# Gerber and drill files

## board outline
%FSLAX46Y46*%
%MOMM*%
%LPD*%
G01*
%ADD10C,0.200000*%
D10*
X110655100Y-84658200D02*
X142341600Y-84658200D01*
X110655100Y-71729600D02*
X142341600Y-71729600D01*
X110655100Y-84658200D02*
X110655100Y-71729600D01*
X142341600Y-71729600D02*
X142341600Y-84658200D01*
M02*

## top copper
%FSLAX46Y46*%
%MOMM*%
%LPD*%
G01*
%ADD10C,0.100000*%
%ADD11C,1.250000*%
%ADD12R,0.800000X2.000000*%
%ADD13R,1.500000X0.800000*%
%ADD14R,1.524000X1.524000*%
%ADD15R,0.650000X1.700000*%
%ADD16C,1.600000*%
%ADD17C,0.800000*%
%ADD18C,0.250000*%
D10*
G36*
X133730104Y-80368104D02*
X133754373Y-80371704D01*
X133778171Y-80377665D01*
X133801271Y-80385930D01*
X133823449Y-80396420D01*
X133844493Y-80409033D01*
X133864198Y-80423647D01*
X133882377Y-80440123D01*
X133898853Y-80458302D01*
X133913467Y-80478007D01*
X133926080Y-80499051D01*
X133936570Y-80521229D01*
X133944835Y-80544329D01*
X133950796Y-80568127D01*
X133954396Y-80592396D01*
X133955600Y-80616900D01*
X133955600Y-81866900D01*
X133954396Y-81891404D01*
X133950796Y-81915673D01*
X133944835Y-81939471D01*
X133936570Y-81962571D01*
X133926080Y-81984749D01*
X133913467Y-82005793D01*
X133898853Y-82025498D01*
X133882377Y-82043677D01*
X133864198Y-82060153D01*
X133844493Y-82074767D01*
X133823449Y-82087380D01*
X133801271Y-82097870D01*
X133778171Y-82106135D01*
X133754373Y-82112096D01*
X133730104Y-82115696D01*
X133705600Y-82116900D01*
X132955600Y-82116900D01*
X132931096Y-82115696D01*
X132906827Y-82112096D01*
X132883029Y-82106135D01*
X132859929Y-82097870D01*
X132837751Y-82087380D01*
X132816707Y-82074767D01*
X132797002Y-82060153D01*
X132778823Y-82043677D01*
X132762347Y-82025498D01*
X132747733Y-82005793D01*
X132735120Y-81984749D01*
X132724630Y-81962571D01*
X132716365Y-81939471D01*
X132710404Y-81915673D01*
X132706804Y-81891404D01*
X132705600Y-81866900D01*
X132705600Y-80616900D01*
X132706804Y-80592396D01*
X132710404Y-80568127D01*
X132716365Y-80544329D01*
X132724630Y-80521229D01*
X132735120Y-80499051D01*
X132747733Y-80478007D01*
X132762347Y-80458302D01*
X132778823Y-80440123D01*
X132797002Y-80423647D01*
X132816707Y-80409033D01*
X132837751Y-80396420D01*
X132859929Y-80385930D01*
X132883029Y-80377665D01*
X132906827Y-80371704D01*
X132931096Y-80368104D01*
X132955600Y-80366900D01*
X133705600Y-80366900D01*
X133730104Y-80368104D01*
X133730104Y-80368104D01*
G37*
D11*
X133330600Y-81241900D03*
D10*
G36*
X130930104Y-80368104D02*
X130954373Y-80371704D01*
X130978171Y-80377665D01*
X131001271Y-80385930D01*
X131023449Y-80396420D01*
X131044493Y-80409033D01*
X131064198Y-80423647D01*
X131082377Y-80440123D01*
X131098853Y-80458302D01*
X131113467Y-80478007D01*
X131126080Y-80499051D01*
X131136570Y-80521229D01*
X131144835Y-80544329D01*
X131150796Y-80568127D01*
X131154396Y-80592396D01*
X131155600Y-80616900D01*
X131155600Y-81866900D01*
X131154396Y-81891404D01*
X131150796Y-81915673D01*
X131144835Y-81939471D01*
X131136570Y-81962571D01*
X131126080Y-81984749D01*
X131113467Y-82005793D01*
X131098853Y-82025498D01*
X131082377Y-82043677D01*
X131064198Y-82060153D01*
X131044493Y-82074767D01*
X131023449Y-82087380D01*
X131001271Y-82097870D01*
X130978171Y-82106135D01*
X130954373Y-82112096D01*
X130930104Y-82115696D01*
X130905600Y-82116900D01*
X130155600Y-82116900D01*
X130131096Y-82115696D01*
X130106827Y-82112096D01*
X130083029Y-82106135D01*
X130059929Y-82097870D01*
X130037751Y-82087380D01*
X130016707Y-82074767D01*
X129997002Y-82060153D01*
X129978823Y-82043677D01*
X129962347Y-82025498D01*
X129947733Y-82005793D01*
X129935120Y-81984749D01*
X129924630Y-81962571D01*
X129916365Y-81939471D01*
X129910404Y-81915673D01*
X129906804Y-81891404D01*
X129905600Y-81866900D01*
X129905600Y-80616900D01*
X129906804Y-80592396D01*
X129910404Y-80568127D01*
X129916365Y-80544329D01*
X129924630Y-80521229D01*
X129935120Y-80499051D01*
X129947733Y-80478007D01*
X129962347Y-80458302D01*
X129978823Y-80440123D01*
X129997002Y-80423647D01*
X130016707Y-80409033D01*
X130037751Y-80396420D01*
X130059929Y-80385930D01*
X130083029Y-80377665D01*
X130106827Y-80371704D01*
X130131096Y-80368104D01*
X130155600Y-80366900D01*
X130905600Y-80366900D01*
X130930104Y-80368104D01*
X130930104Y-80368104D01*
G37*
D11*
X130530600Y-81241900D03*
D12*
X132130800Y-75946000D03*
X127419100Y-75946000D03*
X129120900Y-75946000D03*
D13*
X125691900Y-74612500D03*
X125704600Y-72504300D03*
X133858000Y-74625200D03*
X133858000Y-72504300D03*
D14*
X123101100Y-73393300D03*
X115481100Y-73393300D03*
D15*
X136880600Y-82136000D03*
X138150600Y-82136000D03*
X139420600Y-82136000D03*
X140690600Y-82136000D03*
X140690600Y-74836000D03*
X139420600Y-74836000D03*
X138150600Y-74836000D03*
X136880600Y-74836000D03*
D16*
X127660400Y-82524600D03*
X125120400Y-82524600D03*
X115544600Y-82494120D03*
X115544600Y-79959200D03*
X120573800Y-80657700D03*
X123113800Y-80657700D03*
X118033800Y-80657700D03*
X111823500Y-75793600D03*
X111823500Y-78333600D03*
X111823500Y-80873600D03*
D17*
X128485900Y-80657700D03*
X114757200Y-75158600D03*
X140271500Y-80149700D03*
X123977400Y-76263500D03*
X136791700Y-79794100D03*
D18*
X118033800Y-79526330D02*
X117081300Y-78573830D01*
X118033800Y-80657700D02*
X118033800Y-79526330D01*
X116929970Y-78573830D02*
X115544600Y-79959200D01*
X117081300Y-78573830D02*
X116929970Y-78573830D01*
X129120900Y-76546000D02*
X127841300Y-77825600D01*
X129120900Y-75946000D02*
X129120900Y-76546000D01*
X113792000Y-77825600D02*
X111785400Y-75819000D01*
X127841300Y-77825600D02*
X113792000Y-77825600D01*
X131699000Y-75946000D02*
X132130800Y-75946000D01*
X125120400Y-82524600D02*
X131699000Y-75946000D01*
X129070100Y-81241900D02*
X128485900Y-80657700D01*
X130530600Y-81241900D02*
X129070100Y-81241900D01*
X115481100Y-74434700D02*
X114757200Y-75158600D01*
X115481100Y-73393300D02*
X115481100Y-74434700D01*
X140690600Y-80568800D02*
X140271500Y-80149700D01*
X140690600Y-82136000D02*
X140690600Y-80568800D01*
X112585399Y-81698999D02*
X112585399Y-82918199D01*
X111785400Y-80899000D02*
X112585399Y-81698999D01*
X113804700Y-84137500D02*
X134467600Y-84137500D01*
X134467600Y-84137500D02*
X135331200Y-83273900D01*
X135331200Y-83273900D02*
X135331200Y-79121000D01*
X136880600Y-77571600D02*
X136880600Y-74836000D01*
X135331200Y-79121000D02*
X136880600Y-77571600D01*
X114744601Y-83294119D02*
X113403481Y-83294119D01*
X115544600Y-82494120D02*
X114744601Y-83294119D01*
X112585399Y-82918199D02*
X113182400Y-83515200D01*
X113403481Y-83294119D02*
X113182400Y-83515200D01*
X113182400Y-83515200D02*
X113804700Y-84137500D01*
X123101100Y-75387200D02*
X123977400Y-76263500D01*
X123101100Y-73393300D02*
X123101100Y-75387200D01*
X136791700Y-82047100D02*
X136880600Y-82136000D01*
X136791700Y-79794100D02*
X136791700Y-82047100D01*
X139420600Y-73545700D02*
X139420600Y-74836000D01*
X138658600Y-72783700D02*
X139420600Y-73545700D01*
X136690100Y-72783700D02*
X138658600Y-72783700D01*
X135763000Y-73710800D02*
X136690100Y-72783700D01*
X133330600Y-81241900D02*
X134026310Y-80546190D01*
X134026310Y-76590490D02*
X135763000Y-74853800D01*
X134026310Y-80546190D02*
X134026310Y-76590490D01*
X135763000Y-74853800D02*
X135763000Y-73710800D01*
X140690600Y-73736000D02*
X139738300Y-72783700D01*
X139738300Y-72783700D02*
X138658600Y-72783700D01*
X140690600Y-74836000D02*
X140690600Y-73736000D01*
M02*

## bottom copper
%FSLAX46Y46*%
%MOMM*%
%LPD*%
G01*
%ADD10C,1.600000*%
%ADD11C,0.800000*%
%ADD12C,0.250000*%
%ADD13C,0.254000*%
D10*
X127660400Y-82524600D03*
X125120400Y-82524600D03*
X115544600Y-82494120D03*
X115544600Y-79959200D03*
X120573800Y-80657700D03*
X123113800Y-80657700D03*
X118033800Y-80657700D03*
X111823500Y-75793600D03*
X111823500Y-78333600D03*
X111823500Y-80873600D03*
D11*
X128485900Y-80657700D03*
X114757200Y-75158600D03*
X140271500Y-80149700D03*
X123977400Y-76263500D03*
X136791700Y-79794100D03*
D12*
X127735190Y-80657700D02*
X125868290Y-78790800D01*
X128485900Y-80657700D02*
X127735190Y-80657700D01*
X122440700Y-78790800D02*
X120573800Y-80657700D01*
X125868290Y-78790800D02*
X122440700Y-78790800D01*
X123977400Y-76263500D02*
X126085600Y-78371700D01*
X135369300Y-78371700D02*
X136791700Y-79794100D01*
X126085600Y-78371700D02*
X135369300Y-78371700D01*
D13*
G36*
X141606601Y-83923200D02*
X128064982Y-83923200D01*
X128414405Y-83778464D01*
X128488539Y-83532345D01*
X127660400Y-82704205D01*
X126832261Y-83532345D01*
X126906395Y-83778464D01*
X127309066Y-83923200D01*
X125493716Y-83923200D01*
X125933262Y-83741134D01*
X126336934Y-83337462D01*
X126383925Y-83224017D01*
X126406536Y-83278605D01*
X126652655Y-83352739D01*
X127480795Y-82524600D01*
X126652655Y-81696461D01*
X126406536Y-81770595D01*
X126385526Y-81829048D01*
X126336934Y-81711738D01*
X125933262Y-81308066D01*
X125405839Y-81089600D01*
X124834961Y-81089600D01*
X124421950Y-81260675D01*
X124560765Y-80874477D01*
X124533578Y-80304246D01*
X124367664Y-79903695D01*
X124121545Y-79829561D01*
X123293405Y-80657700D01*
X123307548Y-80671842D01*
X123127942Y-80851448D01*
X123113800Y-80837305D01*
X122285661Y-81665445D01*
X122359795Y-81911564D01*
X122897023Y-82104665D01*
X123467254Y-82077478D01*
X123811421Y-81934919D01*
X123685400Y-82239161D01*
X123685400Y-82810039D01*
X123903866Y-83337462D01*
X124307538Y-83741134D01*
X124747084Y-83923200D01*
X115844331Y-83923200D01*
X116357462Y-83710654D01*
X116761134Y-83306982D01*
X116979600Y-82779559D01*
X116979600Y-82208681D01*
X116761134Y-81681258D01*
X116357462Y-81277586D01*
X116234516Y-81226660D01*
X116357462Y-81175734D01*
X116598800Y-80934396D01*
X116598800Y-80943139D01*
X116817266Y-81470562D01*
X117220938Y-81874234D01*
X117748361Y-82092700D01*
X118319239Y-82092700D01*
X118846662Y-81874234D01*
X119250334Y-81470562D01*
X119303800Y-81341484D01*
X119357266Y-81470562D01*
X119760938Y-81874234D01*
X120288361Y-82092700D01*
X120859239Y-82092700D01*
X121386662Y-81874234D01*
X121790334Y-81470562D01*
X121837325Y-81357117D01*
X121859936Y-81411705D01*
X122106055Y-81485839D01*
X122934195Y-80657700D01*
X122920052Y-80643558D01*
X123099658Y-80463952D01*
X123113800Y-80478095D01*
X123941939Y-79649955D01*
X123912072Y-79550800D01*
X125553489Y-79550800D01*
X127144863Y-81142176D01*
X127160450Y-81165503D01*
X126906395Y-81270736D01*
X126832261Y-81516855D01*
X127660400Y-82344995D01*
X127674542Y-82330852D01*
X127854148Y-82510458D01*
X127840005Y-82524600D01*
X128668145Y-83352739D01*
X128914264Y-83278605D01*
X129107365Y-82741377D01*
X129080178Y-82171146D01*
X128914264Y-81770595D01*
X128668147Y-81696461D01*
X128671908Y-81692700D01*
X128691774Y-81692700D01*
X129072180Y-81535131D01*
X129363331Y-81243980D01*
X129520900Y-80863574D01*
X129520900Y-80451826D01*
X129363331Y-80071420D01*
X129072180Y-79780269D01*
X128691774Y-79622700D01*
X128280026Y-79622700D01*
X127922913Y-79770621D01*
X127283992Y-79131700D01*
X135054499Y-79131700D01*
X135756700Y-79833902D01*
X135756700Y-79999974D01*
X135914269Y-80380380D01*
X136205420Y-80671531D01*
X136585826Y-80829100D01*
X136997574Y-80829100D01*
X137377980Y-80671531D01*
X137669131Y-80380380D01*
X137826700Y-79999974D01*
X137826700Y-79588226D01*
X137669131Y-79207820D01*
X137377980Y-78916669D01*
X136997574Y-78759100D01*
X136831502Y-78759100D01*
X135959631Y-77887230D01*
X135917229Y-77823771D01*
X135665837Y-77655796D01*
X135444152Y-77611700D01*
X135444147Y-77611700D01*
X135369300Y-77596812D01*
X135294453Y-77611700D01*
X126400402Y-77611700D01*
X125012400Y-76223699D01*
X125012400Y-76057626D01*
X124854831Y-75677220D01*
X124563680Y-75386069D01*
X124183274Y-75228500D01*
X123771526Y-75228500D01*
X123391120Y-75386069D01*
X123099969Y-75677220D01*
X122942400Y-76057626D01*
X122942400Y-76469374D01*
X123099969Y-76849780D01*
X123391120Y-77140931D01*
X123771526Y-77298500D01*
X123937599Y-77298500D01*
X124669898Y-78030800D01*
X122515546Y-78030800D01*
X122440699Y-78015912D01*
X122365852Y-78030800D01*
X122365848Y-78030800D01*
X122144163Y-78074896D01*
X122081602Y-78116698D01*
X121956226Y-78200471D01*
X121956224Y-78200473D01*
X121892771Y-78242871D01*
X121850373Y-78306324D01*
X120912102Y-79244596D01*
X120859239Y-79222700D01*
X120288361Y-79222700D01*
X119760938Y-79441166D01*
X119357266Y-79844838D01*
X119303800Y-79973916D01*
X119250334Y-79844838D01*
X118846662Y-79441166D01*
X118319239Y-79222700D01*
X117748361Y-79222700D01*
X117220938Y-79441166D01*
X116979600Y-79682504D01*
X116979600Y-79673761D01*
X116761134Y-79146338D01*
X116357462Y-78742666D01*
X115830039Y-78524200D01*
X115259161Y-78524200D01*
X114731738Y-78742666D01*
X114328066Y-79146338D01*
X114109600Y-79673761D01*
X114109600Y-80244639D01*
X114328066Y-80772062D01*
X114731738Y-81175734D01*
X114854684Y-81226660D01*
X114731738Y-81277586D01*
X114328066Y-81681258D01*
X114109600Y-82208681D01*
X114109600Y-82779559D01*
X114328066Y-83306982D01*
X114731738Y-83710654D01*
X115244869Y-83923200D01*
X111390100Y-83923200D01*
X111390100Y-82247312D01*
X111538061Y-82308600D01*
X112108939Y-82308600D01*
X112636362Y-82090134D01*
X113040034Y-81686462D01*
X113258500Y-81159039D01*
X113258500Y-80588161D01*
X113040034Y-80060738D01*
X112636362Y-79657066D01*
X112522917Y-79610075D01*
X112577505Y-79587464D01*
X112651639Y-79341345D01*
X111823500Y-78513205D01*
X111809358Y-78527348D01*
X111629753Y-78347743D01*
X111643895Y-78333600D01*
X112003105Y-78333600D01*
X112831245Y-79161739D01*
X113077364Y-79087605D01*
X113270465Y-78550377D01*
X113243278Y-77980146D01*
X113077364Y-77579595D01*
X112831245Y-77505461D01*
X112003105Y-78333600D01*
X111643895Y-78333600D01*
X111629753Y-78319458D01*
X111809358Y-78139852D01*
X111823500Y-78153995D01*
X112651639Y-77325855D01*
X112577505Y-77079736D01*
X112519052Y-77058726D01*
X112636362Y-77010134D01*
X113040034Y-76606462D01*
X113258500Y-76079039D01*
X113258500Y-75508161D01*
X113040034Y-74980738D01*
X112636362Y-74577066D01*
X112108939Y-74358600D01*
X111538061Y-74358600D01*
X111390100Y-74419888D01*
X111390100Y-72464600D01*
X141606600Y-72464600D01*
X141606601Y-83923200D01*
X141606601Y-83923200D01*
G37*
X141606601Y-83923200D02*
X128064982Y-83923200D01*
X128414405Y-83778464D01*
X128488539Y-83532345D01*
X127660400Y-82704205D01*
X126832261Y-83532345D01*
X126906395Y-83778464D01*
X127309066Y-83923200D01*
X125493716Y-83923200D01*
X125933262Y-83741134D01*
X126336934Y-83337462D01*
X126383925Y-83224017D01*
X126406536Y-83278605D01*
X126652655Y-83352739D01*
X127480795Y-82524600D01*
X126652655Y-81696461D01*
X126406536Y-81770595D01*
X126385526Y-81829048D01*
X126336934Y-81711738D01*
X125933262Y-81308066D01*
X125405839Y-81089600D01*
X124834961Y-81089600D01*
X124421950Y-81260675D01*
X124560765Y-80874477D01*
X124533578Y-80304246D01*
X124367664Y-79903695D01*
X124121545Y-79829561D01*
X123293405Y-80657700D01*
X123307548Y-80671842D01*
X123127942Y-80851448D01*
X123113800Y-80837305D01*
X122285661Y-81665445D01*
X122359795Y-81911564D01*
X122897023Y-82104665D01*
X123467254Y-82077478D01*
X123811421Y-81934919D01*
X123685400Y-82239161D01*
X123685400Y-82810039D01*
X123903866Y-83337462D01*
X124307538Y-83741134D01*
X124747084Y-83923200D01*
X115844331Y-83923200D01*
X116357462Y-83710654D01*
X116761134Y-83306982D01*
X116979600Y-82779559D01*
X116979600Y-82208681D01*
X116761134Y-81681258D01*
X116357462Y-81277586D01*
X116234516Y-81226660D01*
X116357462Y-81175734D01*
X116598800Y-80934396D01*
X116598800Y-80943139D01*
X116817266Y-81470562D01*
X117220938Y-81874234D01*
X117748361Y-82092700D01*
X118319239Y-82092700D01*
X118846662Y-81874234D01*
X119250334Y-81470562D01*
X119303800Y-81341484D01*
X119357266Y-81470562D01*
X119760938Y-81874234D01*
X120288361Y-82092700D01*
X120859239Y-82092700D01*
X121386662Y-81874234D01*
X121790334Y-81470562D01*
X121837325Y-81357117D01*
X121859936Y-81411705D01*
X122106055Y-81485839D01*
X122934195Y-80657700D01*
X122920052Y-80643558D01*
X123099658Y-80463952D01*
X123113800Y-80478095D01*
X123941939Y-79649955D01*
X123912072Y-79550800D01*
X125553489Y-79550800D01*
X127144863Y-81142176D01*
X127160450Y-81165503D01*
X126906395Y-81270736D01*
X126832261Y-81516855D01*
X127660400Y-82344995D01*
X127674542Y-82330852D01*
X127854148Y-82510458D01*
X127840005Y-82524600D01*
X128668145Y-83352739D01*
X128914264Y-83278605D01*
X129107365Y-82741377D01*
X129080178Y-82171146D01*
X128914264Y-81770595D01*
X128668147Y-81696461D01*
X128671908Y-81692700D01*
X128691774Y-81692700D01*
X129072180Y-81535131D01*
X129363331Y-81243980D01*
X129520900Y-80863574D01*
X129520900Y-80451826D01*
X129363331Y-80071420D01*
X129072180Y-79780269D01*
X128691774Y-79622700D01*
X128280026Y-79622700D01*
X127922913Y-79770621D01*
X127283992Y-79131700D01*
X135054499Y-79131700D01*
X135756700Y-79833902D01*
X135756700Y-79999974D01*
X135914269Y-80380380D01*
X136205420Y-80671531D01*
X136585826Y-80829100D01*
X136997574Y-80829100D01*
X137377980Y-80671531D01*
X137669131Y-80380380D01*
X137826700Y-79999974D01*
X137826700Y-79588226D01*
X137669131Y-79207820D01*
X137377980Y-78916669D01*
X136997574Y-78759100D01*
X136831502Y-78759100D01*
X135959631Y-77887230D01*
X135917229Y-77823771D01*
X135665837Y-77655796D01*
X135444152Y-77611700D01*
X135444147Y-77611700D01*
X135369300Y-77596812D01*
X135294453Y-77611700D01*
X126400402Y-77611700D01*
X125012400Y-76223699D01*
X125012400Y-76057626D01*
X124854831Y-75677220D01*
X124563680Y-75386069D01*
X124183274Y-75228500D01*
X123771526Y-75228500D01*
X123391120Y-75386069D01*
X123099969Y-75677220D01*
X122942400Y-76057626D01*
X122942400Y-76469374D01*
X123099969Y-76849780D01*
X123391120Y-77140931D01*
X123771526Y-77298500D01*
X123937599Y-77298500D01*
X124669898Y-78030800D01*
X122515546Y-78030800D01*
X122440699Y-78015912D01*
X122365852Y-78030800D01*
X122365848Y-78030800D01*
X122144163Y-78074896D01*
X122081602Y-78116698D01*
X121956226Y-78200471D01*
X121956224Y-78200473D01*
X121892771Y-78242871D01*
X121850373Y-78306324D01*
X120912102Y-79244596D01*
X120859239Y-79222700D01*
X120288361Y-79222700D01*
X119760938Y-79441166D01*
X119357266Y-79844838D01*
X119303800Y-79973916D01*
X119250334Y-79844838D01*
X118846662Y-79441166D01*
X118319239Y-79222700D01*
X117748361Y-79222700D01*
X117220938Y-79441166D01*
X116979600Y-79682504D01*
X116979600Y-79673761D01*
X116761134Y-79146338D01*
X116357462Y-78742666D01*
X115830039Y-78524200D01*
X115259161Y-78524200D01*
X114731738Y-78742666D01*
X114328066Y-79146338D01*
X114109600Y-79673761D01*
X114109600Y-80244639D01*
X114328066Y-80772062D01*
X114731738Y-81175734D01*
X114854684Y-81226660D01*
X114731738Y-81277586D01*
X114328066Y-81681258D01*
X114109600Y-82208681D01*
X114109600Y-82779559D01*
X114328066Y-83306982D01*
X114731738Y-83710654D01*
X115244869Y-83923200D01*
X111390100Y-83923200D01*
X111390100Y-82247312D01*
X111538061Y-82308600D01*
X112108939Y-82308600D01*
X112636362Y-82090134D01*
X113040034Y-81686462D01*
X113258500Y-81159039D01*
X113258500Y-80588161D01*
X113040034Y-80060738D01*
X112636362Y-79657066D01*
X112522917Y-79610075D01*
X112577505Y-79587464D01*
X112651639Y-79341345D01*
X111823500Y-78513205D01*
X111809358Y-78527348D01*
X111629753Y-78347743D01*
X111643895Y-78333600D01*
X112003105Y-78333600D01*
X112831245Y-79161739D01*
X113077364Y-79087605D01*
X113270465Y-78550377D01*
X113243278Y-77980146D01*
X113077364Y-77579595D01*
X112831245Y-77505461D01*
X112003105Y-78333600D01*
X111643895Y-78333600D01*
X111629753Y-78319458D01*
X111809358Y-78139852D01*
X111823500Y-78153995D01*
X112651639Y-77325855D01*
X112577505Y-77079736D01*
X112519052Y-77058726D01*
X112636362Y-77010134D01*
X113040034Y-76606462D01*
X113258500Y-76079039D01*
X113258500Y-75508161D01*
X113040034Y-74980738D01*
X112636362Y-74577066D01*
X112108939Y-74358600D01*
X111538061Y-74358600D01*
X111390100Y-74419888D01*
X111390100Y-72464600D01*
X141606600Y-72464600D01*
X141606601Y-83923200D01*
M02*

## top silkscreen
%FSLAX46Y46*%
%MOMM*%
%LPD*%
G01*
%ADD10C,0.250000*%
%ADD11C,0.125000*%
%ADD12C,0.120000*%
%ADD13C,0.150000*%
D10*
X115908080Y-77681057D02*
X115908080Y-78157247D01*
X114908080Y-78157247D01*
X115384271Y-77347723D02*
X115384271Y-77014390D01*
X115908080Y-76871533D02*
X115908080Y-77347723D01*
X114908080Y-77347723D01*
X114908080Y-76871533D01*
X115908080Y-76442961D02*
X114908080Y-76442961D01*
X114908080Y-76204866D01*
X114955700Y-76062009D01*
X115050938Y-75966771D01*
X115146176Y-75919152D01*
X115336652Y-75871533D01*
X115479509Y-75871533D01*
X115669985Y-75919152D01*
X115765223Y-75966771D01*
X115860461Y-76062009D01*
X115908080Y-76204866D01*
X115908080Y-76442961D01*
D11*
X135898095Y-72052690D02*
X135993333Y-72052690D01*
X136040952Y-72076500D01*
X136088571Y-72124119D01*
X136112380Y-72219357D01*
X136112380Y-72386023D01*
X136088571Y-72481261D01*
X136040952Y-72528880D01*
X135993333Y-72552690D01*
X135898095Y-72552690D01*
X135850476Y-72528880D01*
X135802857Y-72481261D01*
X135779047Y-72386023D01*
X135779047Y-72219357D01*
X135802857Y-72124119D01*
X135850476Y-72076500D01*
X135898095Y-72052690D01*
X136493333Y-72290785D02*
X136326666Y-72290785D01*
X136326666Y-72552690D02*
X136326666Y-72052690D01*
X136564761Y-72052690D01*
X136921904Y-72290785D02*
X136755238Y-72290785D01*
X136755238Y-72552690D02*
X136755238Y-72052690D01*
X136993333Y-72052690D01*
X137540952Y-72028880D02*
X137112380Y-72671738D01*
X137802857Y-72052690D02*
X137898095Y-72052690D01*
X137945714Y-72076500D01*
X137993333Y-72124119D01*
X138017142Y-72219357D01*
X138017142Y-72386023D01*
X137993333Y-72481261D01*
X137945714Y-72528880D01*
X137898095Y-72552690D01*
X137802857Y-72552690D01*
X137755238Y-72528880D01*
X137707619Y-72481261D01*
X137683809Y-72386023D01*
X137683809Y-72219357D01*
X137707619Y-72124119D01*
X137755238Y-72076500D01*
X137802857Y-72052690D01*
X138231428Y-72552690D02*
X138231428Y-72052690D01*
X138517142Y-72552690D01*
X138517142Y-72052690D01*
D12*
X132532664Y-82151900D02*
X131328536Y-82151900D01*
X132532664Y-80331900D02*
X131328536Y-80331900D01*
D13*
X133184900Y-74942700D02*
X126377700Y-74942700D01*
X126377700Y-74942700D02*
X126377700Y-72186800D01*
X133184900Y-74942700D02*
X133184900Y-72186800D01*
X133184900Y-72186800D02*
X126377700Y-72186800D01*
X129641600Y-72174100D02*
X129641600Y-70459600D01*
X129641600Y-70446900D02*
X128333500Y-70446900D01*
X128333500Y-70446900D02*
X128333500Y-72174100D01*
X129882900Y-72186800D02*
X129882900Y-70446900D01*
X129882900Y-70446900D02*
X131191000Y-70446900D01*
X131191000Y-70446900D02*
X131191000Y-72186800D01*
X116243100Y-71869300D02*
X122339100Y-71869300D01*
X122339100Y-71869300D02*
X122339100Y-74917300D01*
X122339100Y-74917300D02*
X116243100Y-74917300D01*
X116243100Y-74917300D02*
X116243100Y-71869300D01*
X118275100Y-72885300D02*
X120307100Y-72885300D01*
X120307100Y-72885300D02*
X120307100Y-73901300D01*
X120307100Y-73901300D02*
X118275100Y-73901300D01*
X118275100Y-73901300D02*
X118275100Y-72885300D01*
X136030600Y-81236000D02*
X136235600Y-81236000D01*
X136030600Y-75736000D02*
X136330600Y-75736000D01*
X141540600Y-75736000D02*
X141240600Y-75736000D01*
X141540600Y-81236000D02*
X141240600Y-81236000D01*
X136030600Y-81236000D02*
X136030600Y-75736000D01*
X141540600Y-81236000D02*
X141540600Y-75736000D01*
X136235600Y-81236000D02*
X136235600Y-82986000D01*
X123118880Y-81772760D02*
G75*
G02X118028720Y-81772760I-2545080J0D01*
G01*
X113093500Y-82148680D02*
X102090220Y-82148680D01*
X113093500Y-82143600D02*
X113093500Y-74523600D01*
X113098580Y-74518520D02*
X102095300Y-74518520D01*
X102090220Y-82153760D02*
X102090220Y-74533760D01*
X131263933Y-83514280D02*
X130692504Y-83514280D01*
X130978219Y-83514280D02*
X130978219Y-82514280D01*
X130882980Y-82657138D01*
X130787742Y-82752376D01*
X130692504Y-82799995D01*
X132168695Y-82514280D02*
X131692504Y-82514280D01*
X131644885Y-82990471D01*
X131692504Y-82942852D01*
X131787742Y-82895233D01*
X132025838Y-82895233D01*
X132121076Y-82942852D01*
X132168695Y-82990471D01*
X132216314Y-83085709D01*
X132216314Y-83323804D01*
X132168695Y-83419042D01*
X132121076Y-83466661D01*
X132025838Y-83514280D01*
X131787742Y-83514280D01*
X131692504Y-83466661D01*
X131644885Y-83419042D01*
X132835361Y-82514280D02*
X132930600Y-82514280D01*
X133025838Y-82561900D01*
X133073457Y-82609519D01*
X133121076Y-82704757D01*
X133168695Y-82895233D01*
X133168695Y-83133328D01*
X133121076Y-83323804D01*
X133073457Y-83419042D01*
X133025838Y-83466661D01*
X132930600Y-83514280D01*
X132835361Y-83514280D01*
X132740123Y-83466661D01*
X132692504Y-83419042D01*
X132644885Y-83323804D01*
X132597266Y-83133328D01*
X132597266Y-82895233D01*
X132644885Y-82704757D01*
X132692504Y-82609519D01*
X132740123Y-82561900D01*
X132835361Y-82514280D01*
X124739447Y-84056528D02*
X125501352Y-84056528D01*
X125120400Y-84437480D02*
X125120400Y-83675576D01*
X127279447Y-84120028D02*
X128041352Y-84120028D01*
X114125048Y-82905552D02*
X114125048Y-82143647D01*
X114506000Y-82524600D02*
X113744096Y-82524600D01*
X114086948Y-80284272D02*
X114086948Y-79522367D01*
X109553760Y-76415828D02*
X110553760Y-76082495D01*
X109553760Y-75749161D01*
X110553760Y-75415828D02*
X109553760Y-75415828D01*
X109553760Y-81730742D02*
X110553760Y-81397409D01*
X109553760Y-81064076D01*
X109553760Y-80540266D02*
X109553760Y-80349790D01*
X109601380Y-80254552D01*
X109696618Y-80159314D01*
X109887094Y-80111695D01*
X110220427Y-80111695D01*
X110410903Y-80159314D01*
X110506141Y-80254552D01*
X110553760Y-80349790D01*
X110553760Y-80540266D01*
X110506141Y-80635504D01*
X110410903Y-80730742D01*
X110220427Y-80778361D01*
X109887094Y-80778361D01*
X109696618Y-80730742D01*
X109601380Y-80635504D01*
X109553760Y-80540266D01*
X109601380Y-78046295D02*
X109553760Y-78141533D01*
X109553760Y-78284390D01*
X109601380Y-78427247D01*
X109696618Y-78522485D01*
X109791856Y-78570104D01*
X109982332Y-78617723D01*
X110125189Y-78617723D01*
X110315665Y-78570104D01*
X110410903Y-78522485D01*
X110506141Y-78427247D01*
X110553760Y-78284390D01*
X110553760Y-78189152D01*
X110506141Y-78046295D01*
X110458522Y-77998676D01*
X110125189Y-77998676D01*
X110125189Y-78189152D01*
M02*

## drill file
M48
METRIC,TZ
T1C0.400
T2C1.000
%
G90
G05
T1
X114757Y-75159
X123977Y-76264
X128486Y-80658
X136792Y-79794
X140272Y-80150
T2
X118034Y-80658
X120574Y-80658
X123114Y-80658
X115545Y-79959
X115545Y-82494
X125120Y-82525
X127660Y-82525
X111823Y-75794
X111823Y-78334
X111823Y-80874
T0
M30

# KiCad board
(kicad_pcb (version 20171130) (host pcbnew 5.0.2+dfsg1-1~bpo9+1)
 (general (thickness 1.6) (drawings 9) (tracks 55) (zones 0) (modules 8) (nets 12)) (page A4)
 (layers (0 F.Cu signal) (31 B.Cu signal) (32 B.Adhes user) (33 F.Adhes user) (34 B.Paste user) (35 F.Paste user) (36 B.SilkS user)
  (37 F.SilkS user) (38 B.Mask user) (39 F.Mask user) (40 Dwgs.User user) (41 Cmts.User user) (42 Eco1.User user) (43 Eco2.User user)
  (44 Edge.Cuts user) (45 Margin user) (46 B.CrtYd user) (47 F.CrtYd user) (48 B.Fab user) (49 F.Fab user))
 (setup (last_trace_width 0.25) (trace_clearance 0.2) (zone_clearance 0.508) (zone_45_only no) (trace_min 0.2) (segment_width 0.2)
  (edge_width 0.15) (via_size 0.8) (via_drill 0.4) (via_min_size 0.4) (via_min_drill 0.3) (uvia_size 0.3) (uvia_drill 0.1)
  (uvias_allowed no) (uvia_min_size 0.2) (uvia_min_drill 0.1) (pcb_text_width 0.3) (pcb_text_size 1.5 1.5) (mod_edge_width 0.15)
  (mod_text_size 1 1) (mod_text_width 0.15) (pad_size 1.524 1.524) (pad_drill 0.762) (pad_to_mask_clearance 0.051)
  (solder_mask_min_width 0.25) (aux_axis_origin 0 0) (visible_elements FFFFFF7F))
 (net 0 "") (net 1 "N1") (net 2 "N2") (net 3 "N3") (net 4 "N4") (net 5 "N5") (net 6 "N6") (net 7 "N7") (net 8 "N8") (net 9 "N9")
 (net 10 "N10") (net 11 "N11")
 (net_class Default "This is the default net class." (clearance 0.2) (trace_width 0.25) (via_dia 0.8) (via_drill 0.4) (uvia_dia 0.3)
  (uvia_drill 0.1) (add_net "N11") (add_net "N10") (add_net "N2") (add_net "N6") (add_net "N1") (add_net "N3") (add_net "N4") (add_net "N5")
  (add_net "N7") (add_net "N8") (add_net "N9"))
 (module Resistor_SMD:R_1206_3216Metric (layer F.Cu) (at 131.9306 81.2419 180)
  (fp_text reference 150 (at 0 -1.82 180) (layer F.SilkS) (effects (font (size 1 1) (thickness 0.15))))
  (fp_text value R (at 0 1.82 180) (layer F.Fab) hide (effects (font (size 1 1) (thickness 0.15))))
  (fp_line (start -0.602064 -0.91) (end 0.602064 -0.91) (layer F.SilkS) (width 0.12))
  (fp_line (start -0.602064 0.91) (end 0.602064 0.91) (layer F.SilkS) (width 0.12))
  (pad 1 smd roundrect (at -1.4 0 180) (size 1.25 1.75) (layers F.Cu F.Paste F.Mask) (roundrect_rratio 0.2) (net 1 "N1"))
  (pad 2 smd roundrect (at 1.4 0 180) (size 1.25 1.75) (layers F.Cu F.Paste F.Mask) (roundrect_rratio 0.2) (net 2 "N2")))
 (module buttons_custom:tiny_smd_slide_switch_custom (layer F.Cu) (at 132.1308 74.9427 180)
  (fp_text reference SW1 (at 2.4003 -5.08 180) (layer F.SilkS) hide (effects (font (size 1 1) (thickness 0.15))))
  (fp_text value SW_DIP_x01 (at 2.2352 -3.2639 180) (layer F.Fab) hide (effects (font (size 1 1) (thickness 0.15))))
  (fp_line (start -1.0541 0) (end 5.7531 0) (layer F.SilkS) (width 0.15))
  (fp_line (start 5.7531 0) (end 5.7531 2.7559) (layer F.SilkS) (width 0.15))
  (fp_line (start -1.0541 0) (end -1.0541 2.7559) (layer F.SilkS) (width 0.15))
  (fp_line (start -1.0541 2.7559) (end 5.7531 2.7559) (layer F.SilkS) (width 0.15))
  (fp_line (start 2.4892 2.7686) (end 2.4892 4.4831) (layer F.SilkS) (width 0.15))
  (fp_line (start 2.4892 4.4958) (end 3.7973 4.4958) (layer F.SilkS) (width 0.15))
  (fp_line (start 3.7973 4.4958) (end 3.7973 2.7686) (layer F.SilkS) (width 0.15))
  (fp_line (start 2.2479 2.7559) (end 2.2479 4.4958) (layer F.SilkS) (width 0.15))
  (fp_line (start 2.2479 4.4958) (end 0.9398 4.4958) (layer F.SilkS) (width 0.15))
  (fp_line (start 0.9398 4.4958) (end 0.9398 2.7559) (layer F.SilkS) (width 0.15))
  (pad 1 smd rect (at 0 -1.0033 180) (size 0.8 2) (layers F.Cu F.Paste F.Mask) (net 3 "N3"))
  (pad 3 smd rect (at 4.7117 -1.0033 180) (size 0.8 2) (layers F.Cu F.Paste F.Mask))
  (pad 2 smd rect (at 3.0099 -1.0033 180) (size 0.8 2) (layers F.Cu F.Paste F.Mask) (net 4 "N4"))
  (pad 4 smd rect (at 6.4389 0.3302 270) (size 0.8 1.5) (layers F.Cu F.Paste F.Mask))
  (pad 4 smd rect (at 6.4262 2.4384 270) (size 0.8 1.5) (layers F.Cu F.Paste F.Mask))
  (pad 4 smd rect (at -1.7272 0.3175 270) (size 0.8 1.5) (layers F.Cu F.Paste F.Mask))
  (pad 4 smd rect (at -1.7272 2.4384 270) (size 0.8 1.5) (layers F.Cu F.Paste F.Mask)))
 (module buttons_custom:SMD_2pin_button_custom (layer F.Cu) (at 119.2911 73.3933)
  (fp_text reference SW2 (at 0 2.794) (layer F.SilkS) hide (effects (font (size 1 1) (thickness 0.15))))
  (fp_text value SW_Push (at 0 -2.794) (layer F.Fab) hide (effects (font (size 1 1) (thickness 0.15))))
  (fp_line (start -3.048 -1.524) (end 3.048 -1.524) (layer F.SilkS) (width 0.15))
  (fp_line (start 3.048 -1.524) (end 3.048 1.524) (layer F.SilkS) (width 0.15))
  (fp_line (start 3.048 1.524) (end -3.048 1.524) (layer F.SilkS) (width 0.15))
  (fp_line (start -3.048 1.524) (end -3.048 -1.524) (layer F.SilkS) (width 0.15))
  (fp_line (start -1.016 -0.508) (end 1.016 -0.508) (layer F.SilkS) (width 0.15))
  (fp_line (start 1.016 -0.508) (end 1.016 0.508) (layer F.SilkS) (width 0.15))
  (fp_line (start 1.016 0.508) (end -1.016 0.508) (layer F.SilkS) (width 0.15))
  (fp_line (start -1.016 0.508) (end -1.016 -0.508) (layer F.SilkS) (width 0.15))
  (pad 1 smd rect (at 3.81 0) (size 1.524 1.524) (layers F.Cu F.Paste F.Mask) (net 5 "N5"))
  (pad 2 smd rect (at -3.81 0) (size 1.524 1.524) (layers F.Cu F.Paste F.Mask) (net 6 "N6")))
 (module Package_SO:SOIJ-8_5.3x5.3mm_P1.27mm (layer F.Cu) (at 138.7856 78.486 90)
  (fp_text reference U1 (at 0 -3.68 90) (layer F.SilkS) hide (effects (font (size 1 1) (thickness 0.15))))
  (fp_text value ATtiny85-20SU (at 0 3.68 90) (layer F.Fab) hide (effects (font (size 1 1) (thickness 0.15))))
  (fp_line (start -2.75 -2.755) (end -2.75 -2.55) (layer F.SilkS) (width 0.15))
  (fp_line (start 2.75 -2.755) (end 2.75 -2.455) (layer F.SilkS) (width 0.15))
  (fp_line (start 2.75 2.755) (end 2.75 2.455) (layer F.SilkS) (width 0.15))
  (fp_line (start -2.75 2.755) (end -2.75 2.455) (layer F.SilkS) (width 0.15))
  (fp_line (start -2.75 -2.755) (end 2.75 -2.755) (layer F.SilkS) (width 0.15))
  (fp_line (start -2.75 2.755) (end 2.75 2.755) (layer F.SilkS) (width 0.15))
  (fp_line (start -2.75 -2.55) (end -4.5 -2.55) (layer F.SilkS) (width 0.15))
  (pad 1 smd rect (at -3.65 -1.905 90) (size 1.7 0.65) (layers F.Cu F.Paste F.Mask) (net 5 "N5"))
  (pad 2 smd rect (at -3.65 -0.635 90) (size 1.7 0.65) (layers F.Cu F.Paste F.Mask) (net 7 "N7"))
  (pad 3 smd rect (at -3.65 0.635 90) (size 1.7 0.65) (layers F.Cu F.Paste F.Mask) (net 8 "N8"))
  (pad 4 smd rect (at -3.65 1.905 90) (size 1.7 0.65) (layers F.Cu F.Paste F.Mask) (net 6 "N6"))
  (pad 5 smd rect (at 3.65 1.905 90) (size 1.7 0.65) (layers F.Cu F.Paste F.Mask) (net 1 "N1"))
  (pad 6 smd rect (at 3.65 0.635 90) (size 1.7 0.65) (layers F.Cu F.Paste F.Mask) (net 1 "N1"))
  (pad 7 smd rect (at 3.65 -0.635 90) (size 1.7 0.65) (layers F.Cu F.Paste F.Mask) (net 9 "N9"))
  (pad 8 smd rect (at 3.65 -1.905 90) (size 1.7 0.65) (layers F.Cu F.Paste F.Mask) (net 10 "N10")))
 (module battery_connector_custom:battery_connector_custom (layer F.Cu) (at 126.3904 82.5246 180)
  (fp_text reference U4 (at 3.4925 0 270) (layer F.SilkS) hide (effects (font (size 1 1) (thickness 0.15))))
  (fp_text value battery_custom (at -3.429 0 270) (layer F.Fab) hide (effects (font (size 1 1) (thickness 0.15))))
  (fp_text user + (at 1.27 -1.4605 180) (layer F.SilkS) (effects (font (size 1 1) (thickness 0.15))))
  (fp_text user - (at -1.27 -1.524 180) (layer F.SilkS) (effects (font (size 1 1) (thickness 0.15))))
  (pad 1 thru_hole circle (at -1.27 0 180) (size 1.6 1.6) (drill 1) (layers *.Cu *.Mask) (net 6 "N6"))
  (pad 2 thru_hole circle (at 1.27 0 180) (size 1.6 1.6) (drill 1) (layers *.Cu *.Mask) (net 3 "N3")))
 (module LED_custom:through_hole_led (layer F.Cu) (at 115.5446 81.2292 90)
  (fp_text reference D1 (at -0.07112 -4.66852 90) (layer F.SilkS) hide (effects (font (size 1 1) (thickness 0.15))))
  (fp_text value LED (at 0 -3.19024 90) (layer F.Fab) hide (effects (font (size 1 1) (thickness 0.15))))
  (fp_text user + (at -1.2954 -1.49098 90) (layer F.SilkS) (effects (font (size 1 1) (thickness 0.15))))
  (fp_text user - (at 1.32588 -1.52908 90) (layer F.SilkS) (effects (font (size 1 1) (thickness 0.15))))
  (pad 2 thru_hole circle (at -1.26492 0 90) (size 1.6 1.6) (drill 1) (layers *.Cu *.Mask) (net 10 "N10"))
  (pad 1 thru_hole circle (at 1.27 0 90) (size 1.6 1.6) (drill 1) (layers *.Cu *.Mask) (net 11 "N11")))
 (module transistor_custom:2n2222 (layer F.Cu) (at 120.5738 80.6577 180)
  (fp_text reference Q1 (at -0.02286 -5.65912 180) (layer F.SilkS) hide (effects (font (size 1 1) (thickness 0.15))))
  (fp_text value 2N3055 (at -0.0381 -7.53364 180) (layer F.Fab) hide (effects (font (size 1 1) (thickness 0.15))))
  (fp_arc (start 0 -1.11506) (end 2.54508 -1.11506) (angle -180) (layer F.SilkS) (width 0.15))
  (pad 1 thru_hole circle (at 0 0 180) (size 1.6 1.6) (drill 1) (layers *.Cu *.Mask) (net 2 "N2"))
  (pad 2 thru_hole circle (at -2.54 0 180) (size 1.6 1.6) (drill 1) (layers *.Cu *.Mask) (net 6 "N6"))
  (pad 3 thru_hole circle (at 2.54 0 180) (size 1.6 1.6) (drill 1) (layers *.Cu *.Mask) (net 11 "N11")))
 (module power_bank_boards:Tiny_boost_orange (layer F.Cu) (at 111.8235 78.3336 90)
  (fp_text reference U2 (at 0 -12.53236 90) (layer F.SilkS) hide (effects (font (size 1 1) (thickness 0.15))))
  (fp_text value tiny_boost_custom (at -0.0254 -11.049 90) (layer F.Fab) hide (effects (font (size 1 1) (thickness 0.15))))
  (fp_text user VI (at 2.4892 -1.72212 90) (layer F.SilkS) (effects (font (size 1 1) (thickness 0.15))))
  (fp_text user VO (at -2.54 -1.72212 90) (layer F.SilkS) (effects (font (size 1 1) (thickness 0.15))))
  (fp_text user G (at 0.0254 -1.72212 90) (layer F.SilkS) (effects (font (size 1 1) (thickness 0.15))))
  (fp_line (start -3.81508 1.27) (end -3.81508 -9.73328) (layer F.SilkS) (width 0.15))
  (fp_line (start -3.81 1.27) (end 3.81 1.27) (layer F.SilkS) (width 0.15))
  (fp_line (start 3.81508 1.27508) (end 3.81508 -9.7282) (layer F.SilkS) (width 0.15))
  (fp_line (start -3.82016 -9.73328) (end 3.79984 -9.73328) (layer F.SilkS) (width 0.15))
  (pad 1 thru_hole circle (at 2.54 0 90) (size 1.6 1.6) (drill 1) (layers *.Cu *.Mask) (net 4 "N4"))
  (pad 2 thru_hole circle (at 0 0 90) (size 1.6 1.6) (drill 1) (layers *.Cu *.Mask) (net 6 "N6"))
  (pad 3 thru_hole circle (at -2.54 0 90) (size 1.6 1.6) (drill 1) (layers *.Cu *.Mask) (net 10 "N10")))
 (gr_line (start 110.6551 84.6582) (end 142.3416 84.6582) (layer Edge.Cuts) (width 0.2))
 (gr_line (start 110.6551 71.7296) (end 142.3416 71.7296) (layer Edge.Cuts) (width 0.2))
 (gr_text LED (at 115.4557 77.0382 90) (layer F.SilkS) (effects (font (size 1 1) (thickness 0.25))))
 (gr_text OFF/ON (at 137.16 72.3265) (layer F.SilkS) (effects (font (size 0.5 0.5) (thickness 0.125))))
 (gr_line (start 110.6551 84.6582) (end 110.6551 71.7296) (layer Edge.Cuts) (width 0.2))
 (gr_line (start 142.3416 71.7296) (end 142.3416 84.6582) (layer Edge.Cuts) (width 0.2))
 (segment (start 118.0338 79.52633) (end 117.0813 78.57383) (width 0.25) (layer F.Cu) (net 11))
 (segment (start 118.0338 80.6577) (end 118.0338 79.52633) (width 0.25) (layer F.Cu) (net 11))
 (segment (start 116.92997 78.57383) (end 115.5446 79.9592) (width 0.25) (layer F.Cu) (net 11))
 (segment (start 117.0813 78.57383) (end 116.92997 78.57383) (width 0.25) (layer F.Cu) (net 11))
 (segment (start 129.1209 76.546) (end 127.8413 77.8256) (width 0.25) (layer F.Cu) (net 4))
 (segment (start 129.1209 75.946) (end 129.1209 76.546) (width 0.25) (layer F.Cu) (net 4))
 (segment (start 113.792 77.8256) (end 111.7854 75.819) (width 0.25) (layer F.Cu) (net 4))
 (segment (start 127.8413 77.8256) (end 113.792 77.8256) (width 0.25) (layer F.Cu) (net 4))
 (segment (start 131.699 75.946) (end 132.1308 75.946) (width 0.25) (layer F.Cu) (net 3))
 (segment (start 125.1204 82.5246) (end 131.699 75.946) (width 0.25) (layer F.Cu) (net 3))
 (via (at 128.4859 80.6577) (size 0.8) (drill 0.4) (layers F.Cu B.Cu) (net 2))
 (segment (start 129.0701 81.2419) (end 128.4859 80.6577) (width 0.25) (layer F.Cu) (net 2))
 (segment (start 130.5306 81.2419) (end 129.0701 81.2419) (width 0.25) (layer F.Cu) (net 2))
 (segment (start 127.73519 80.6577) (end 125.86829 78.7908) (width 0.25) (layer B.Cu) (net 2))
 (segment (start 128.4859 80.6577) (end 127.73519 80.6577) (width 0.25) (layer B.Cu) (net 2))
 (segment (start 122.4407 78.7908) (end 120.5738 80.6577) (width 0.25) (layer B.Cu) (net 2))
 (segment (start 125.86829 78.7908) (end 122.4407 78.7908) (width 0.25) (layer B.Cu) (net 2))
 (via (at 114.7572 75.1586) (size 0.8) (drill 0.4) (layers F.Cu B.Cu) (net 6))
 (segment (start 115.4811 74.4347) (end 114.7572 75.1586) (width 0.25) (layer F.Cu) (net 6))
 (segment (start 115.4811 73.3933) (end 115.4811 74.4347) (width 0.25) (layer F.Cu) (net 6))
 (via (at 140.2715 80.1497) (size 0.8) (drill 0.4) (layers F.Cu B.Cu) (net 6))
 (segment (start 140.6906 80.5688) (end 140.2715 80.1497) (width 0.25) (layer F.Cu) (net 6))
 (segment (start 140.6906 82.136) (end 140.6906 80.5688) (width 0.25) (layer F.Cu) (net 6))
 (segment (start 112.585399 81.698999) (end 112.585399 82.918199) (width 0.25) (layer F.Cu) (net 10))
 (segment (start 111.7854 80.899) (end 112.585399 81.698999) (width 0.25) (layer F.Cu) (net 10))
 (segment (start 113.8047 84.1375) (end 134.4676 84.1375) (width 0.25) (layer F.Cu) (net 10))
 (segment (start 134.4676 84.1375) (end 135.3312 83.2739) (width 0.25) (layer F.Cu) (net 10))
 (segment (start 135.3312 83.2739) (end 135.3312 79.121) (width 0.25) (layer F.Cu) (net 10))
 (segment (start 136.8806 77.5716) (end 136.8806 74.836) (width 0.25) (layer F.Cu) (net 10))
 (segment (start 135.3312 79.121) (end 136.8806 77.5716) (width 0.25) (layer F.Cu) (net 10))
 (segment (start 114.744601 83.294119) (end 113.403481 83.294119) (width 0.25) (layer F.Cu) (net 10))
 (segment (start 115.5446 82.49412) (end 114.744601 83.294119) (width 0.25) (layer F.Cu) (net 10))
 (segment (start 112.585399 82.918199) (end 113.1824 83.5152) (width 0.25) (layer F.Cu) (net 10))
 (segment (start 113.403481 83.294119) (end 113.1824 83.5152) (width 0.25) (layer F.Cu) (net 10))
 (segment (start 113.1824 83.5152) (end 113.8047 84.1375) (width 0.25) (layer F.Cu) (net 10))
 (via (at 123.9774 76.2635) (size 0.8) (drill 0.4) (layers F.Cu B.Cu) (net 5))
 (segment (start 123.1011 75.3872) (end 123.9774 76.2635) (width 0.25) (layer F.Cu) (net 5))
 (segment (start 123.1011 73.3933) (end 123.1011 75.3872) (width 0.25) (layer F.Cu) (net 5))
 (segment (start 123.9774 76.2635) (end 126.0856 78.3717) (width 0.25) (layer B.Cu) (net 5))
 (via (at 136.7917 79.7941) (size 0.8) (drill 0.4) (layers F.Cu B.Cu) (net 5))
 (segment (start 135.3693 78.3717) (end 136.7917 79.7941) (width 0.25) (layer B.Cu) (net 5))
 (segment (start 126.0856 78.3717) (end 135.3693 78.3717) (width 0.25) (layer B.Cu) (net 5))
 (segment (start 136.7917 82.0471) (end 136.8806 82.136) (width 0.25) (layer F.Cu) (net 5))
 (segment (start 136.7917 79.7941) (end 136.7917 82.0471) (width 0.25) (layer F.Cu) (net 5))
 (segment (start 139.4206 73.5457) (end 139.4206 74.836) (width 0.25) (layer F.Cu) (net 1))
 (segment (start 138.6586 72.7837) (end 139.4206 73.5457) (width 0.25) (layer F.Cu) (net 1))
 (segment (start 136.6901 72.7837) (end 138.6586 72.7837) (width 0.25) (layer F.Cu) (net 1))
 (segment (start 135.763 73.7108) (end 136.6901 72.7837) (width 0.25) (layer F.Cu) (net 1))
 (segment (start 133.3306 81.2419) (end 134.02631 80.54619) (width 0.25) (layer F.Cu) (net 1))
 (segment (start 134.02631 76.59049) (end 135.763 74.8538) (width 0.25) (layer F.Cu) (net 1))
 (segment (start 134.02631 80.54619) (end 134.02631 76.59049) (width 0.25) (layer F.Cu) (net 1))
 (segment (start 135.763 74.8538) (end 135.763 73.7108) (width 0.25) (layer F.Cu) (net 1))
 (segment (start 140.6906 73.736) (end 139.7383 72.7837) (width 0.25) (layer F.Cu) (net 1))
 (segment (start 139.7383 72.7837) (end 138.6586 72.7837) (width 0.25) (layer F.Cu) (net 1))
 (segment (start 140.6906 74.836) (end 140.6906 73.736) (width 0.25) (layer F.Cu) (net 1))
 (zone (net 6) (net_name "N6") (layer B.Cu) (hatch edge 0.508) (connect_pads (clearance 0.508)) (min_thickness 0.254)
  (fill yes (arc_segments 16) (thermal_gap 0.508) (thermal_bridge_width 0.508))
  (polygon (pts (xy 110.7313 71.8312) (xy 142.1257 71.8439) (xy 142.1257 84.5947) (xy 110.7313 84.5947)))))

